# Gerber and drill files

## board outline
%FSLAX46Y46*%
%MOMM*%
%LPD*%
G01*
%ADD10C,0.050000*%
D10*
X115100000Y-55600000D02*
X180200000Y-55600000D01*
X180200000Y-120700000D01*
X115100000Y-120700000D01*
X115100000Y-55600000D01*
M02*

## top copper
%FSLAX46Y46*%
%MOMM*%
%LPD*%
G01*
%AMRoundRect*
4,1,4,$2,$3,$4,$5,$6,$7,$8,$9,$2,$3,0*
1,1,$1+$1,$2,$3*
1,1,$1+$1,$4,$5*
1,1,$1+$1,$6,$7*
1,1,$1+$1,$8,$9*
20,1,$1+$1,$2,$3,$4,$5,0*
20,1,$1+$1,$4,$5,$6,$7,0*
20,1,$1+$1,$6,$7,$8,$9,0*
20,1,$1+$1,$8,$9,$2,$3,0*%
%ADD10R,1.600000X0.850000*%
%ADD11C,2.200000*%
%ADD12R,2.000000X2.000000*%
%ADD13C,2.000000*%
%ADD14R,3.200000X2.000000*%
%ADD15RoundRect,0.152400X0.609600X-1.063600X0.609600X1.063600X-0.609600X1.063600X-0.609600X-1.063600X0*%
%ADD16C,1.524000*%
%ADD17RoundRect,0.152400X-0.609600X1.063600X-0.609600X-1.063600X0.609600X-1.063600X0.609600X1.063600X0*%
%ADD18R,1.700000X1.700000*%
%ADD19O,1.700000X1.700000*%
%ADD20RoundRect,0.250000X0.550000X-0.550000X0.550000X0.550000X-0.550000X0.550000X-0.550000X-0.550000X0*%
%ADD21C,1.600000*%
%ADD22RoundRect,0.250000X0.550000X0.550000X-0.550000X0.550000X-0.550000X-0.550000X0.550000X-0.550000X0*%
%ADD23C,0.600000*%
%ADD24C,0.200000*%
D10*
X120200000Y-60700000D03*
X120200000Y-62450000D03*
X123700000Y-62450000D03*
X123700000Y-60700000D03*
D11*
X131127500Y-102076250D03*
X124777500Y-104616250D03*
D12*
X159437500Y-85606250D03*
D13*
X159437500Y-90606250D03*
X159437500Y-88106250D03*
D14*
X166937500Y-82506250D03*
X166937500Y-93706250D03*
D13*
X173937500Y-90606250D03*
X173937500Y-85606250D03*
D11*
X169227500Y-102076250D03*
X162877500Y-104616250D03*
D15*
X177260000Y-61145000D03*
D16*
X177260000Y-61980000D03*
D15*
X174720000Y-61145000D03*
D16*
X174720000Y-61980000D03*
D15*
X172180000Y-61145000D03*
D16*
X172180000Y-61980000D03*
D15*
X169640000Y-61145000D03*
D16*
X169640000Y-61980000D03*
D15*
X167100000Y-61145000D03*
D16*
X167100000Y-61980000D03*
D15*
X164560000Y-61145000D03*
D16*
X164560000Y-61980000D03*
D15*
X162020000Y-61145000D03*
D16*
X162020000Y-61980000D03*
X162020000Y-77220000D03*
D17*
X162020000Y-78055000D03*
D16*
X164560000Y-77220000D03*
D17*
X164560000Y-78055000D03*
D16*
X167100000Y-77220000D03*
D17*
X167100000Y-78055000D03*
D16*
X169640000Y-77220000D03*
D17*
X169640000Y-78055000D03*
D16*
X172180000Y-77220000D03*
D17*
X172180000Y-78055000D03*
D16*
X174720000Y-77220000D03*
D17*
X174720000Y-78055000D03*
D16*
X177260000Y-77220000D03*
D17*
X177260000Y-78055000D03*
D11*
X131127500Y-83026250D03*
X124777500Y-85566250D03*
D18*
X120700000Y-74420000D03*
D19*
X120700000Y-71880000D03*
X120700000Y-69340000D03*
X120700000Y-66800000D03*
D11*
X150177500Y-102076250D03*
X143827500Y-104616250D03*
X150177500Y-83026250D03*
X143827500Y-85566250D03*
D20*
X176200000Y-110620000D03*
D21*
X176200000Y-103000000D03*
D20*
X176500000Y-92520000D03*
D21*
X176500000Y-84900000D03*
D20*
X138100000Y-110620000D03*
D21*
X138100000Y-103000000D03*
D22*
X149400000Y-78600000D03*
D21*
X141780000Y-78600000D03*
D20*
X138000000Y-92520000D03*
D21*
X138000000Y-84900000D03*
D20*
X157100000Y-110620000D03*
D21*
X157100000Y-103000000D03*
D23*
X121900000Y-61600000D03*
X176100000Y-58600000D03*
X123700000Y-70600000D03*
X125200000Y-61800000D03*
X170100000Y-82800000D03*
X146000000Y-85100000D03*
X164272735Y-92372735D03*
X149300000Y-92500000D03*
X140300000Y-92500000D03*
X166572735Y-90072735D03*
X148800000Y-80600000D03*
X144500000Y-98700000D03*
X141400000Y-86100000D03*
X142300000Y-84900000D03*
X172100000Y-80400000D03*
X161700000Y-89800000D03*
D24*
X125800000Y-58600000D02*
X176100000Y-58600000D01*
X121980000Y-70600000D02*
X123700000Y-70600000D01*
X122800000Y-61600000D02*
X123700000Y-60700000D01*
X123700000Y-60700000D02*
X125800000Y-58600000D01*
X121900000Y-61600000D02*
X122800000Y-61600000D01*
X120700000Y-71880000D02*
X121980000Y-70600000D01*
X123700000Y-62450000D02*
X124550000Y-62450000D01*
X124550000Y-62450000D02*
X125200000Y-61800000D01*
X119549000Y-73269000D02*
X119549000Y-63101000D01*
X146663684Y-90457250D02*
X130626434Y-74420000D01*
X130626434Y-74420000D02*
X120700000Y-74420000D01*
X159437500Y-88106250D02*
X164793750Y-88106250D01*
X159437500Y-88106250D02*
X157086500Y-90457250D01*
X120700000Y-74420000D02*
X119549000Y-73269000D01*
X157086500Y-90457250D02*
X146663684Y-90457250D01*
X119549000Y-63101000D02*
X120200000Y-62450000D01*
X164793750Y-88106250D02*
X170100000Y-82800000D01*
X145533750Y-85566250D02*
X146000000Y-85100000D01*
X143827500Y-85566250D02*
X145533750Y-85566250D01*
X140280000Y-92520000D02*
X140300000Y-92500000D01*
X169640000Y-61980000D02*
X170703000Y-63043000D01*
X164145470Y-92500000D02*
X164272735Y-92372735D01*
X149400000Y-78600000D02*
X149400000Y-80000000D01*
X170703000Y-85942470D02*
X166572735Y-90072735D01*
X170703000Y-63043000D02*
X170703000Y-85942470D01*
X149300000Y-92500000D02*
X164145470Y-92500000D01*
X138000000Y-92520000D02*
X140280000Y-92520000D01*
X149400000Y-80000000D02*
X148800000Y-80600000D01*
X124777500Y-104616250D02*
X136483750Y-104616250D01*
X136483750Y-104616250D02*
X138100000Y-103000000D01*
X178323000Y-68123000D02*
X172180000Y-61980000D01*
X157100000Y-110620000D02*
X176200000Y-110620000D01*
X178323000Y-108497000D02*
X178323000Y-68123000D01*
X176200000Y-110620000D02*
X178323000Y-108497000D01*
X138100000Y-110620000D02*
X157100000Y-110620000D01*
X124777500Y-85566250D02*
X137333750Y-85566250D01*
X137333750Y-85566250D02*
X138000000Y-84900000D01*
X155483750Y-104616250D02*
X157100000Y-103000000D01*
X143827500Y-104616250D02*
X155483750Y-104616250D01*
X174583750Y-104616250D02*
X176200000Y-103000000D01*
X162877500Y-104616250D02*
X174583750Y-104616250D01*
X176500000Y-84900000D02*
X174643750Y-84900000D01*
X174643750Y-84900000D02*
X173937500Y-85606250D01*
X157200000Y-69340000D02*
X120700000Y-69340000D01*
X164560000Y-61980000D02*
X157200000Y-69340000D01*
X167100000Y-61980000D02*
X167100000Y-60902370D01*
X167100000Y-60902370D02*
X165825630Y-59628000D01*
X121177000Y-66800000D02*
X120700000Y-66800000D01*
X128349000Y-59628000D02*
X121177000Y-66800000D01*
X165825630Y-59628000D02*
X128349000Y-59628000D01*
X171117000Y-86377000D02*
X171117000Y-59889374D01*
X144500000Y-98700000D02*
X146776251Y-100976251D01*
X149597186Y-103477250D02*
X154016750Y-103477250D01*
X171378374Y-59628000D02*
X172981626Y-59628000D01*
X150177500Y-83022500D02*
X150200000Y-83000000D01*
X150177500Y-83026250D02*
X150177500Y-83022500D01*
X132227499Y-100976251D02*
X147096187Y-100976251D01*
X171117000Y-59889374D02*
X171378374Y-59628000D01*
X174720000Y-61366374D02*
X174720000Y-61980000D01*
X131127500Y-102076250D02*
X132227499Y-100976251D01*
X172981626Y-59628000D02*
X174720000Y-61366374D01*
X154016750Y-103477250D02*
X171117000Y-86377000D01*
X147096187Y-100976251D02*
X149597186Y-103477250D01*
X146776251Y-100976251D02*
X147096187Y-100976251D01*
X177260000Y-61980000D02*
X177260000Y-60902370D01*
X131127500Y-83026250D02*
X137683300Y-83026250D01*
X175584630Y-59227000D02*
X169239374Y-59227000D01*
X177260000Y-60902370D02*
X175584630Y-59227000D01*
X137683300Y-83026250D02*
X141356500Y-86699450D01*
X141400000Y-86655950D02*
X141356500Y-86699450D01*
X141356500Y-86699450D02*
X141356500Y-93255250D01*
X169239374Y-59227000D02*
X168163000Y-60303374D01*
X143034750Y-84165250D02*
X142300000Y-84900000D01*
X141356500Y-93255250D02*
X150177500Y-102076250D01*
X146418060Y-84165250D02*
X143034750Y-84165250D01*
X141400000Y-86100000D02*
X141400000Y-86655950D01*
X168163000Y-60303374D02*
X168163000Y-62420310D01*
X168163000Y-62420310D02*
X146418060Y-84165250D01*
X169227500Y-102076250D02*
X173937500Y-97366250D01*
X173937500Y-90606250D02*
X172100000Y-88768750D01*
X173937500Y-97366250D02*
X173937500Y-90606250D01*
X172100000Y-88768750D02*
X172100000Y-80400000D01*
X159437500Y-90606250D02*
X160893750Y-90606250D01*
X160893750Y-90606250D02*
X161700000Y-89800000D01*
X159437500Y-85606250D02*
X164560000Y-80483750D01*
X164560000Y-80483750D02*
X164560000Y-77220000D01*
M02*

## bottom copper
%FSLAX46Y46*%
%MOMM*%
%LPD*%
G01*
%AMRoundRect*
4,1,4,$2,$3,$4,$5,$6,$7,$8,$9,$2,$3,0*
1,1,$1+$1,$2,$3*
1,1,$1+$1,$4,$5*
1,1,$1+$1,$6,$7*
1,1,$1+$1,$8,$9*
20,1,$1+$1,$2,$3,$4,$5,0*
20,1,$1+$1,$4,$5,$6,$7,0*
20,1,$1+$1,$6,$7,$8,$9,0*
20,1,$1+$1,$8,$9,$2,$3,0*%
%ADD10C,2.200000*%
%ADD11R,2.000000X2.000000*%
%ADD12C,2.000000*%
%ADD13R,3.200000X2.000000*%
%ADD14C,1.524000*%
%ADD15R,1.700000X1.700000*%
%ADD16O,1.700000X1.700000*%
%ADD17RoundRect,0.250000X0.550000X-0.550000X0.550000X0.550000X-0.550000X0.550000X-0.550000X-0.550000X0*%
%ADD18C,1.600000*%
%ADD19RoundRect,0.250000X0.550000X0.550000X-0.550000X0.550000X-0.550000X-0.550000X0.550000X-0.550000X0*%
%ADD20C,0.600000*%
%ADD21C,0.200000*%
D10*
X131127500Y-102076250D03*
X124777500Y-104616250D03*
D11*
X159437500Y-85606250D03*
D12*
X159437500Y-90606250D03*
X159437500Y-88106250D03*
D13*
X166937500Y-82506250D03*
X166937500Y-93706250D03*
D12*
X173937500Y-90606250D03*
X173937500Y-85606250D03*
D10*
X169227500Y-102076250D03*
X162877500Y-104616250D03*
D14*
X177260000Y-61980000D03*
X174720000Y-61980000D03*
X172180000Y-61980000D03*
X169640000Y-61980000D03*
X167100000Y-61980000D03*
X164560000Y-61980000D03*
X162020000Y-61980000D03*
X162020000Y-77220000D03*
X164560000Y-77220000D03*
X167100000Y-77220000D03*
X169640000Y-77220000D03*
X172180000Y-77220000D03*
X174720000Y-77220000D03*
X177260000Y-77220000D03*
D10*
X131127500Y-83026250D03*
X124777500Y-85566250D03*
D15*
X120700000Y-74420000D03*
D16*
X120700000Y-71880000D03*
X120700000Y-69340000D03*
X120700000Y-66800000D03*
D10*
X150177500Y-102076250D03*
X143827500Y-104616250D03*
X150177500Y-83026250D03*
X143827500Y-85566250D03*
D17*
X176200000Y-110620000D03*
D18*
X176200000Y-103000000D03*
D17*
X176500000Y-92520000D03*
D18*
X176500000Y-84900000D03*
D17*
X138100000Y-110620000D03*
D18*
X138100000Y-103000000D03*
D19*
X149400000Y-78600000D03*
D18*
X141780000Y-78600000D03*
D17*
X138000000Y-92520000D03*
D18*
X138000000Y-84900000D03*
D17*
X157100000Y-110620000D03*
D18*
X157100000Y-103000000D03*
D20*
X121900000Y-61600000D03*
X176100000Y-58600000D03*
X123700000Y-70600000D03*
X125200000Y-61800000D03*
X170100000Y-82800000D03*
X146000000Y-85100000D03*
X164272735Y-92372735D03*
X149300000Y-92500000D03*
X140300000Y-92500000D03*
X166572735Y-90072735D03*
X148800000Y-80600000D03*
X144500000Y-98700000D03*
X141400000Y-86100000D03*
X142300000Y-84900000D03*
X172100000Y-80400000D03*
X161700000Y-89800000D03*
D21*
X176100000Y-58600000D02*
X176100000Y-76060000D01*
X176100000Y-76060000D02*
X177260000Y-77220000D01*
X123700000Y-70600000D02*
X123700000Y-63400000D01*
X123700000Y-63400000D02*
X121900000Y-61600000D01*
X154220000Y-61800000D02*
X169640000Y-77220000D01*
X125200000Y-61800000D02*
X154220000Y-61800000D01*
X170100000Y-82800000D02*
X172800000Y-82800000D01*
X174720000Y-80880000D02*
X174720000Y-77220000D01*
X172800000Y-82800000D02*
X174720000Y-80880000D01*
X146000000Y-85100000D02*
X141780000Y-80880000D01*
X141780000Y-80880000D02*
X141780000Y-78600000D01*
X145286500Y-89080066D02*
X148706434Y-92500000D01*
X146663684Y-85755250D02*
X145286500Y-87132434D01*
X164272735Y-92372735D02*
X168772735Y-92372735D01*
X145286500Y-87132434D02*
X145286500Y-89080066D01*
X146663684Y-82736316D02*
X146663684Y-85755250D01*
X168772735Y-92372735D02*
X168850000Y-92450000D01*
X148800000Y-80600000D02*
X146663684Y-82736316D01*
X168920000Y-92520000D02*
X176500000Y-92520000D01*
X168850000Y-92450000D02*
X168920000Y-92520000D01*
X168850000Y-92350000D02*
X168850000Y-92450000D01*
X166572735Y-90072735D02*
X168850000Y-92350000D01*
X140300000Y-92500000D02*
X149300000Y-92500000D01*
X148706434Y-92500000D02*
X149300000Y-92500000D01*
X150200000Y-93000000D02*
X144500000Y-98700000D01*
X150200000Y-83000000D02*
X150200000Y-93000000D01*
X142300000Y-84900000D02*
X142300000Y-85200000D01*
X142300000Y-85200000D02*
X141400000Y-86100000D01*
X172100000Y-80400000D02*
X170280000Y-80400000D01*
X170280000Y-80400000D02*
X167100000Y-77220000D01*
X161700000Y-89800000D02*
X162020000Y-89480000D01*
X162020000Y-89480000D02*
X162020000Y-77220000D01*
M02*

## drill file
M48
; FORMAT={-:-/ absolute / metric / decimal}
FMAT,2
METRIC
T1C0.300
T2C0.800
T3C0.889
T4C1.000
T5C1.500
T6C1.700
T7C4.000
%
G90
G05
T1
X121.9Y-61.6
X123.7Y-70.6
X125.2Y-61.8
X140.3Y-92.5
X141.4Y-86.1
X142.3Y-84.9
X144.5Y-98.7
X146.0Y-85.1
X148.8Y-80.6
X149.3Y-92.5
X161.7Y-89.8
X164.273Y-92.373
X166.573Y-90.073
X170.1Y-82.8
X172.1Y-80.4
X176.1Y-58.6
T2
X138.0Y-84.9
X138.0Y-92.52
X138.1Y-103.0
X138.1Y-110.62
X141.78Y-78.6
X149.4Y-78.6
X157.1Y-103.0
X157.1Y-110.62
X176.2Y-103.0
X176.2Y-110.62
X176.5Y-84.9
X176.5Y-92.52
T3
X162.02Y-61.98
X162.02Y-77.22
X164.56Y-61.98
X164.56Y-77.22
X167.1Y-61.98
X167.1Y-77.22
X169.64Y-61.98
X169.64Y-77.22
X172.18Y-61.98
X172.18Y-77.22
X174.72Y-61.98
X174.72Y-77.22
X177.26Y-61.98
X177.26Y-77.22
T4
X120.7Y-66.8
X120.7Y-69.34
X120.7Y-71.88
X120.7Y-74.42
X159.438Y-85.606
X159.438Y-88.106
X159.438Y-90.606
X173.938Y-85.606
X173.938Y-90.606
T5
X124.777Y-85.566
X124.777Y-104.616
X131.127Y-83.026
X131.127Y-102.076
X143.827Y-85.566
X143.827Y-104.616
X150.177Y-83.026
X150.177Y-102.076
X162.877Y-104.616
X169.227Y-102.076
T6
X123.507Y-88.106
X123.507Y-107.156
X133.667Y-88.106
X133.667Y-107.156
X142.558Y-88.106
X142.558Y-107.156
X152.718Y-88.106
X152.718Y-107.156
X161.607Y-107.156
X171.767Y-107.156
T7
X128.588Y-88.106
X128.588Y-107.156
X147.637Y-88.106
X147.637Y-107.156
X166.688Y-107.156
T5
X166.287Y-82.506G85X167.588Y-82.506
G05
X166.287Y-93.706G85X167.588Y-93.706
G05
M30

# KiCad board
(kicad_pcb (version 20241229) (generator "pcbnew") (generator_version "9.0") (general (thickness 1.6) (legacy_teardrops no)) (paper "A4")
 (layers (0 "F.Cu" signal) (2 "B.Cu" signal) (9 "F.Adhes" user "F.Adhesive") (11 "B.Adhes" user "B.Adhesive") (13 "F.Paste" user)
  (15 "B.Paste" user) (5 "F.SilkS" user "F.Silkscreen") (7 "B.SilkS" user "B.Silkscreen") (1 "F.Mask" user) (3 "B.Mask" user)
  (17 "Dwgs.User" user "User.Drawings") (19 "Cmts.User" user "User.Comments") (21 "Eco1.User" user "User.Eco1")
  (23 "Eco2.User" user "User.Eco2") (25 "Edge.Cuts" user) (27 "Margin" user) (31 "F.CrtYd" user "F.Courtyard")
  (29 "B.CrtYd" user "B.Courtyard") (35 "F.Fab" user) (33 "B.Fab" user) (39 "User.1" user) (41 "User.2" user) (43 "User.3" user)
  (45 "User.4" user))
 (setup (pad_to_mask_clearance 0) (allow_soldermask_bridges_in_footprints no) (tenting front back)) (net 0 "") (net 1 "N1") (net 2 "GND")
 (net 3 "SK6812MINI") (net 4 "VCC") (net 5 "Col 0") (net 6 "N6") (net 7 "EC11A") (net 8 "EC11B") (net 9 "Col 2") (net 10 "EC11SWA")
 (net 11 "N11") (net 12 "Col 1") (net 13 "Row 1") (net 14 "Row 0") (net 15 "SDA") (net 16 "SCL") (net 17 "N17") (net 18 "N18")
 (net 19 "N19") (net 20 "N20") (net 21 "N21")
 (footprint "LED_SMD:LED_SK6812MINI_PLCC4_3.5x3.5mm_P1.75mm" (layer "F.Cu") (at 121.95 61.575)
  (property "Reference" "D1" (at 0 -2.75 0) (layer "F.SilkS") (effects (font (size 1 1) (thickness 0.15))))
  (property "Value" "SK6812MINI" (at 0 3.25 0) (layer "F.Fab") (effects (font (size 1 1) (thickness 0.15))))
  (pad "1" smd rect (at -1.75 -0.875) (size 1.6 0.85) (layers "F.Cu" "F.Mask" "F.Paste") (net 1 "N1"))
  (pad "2" smd rect (at -1.75 0.875) (size 1.6 0.85) (layers "F.Cu" "F.Mask" "F.Paste") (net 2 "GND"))
  (pad "3" smd rect (at 1.75 0.875) (size 1.6 0.85) (layers "F.Cu" "F.Mask" "F.Paste") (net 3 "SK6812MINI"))
  (pad "4" smd rect (at 1.75 -0.875) (size 1.6 0.85) (layers "F.Cu" "F.Mask" "F.Paste") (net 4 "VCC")))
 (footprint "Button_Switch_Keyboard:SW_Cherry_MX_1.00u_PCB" (layer "F.Cu") (at 131.1275 102.07625)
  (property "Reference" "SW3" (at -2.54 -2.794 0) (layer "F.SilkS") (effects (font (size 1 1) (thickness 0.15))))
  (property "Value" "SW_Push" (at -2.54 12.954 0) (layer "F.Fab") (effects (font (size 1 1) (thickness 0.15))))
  (pad "" np_thru_hole circle (at -7.62 5.08) (size 1.7 1.7) (drill 1.7) (layers "*.Cu" "*.Mask"))
  (pad "" np_thru_hole circle (at -2.54 5.08) (size 4 4) (drill 4) (layers "*.Cu" "*.Mask"))
  (pad "" np_thru_hole circle (at 2.54 5.08) (size 1.7 1.7) (drill 1.7) (layers "*.Cu" "*.Mask"))
  (pad "1" thru_hole circle (at 0 0) (size 2.2 2.2) (drill 1.5) (layers "*.Cu" "*.Mask") (remove_unused_layers no) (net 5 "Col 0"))
  (pad "2" thru_hole circle (at -6.35 2.54) (size 2.2 2.2) (drill 1.5) (layers "*.Cu" "*.Mask") (remove_unused_layers no) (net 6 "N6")))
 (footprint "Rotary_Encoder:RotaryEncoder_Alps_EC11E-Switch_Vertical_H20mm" (layer "F.Cu") (at 159.4375 85.60625)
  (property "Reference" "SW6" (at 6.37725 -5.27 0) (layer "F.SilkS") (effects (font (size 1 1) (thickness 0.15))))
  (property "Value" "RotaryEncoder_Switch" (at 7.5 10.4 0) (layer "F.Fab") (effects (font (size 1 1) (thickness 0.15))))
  (pad "A" thru_hole rect (at 0 0) (size 2 2) (drill 1) (layers "*.Cu" "*.Mask") (remove_unused_layers no) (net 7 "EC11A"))
  (pad "B" thru_hole circle (at 0 5) (size 2 2) (drill 1) (layers "*.Cu" "*.Mask") (remove_unused_layers no) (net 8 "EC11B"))
  (pad "C" thru_hole circle (at 0 2.5) (size 2 2) (drill 1) (layers "*.Cu" "*.Mask") (remove_unused_layers no) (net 2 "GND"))
  (pad "MP" thru_hole rect (at 7.5 -3.1) (size 3.2 2) (drill oval 2.8 1.5) (layers "*.Cu" "*.Mask") (remove_unused_layers no))
  (pad "MP" thru_hole rect (at 7.5 8.1) (size 3.2 2) (drill oval 2.8 1.5) (layers "*.Cu" "*.Mask") (remove_unused_layers no))
  (pad "S1" thru_hole circle (at 14.5 5) (size 2 2) (drill 1) (layers "*.Cu" "*.Mask") (remove_unused_layers no) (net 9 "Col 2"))
  (pad "S2" thru_hole circle (at 14.5 0) (size 2 2) (drill 1) (layers "*.Cu" "*.Mask") (remove_unused_layers no) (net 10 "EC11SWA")))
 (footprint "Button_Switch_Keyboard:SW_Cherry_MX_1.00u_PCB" (layer "F.Cu") (at 169.2275 102.07625)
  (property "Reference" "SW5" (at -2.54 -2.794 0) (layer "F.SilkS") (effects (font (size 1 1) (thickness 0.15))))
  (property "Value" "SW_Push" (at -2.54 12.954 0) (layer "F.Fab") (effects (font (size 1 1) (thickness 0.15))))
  (pad "" np_thru_hole circle (at -7.62 5.08) (size 1.7 1.7) (drill 1.7) (layers "*.Cu" "*.Mask"))
  (pad "" np_thru_hole circle (at -2.54 5.08) (size 4 4) (drill 4) (layers "*.Cu" "*.Mask"))
  (pad "" np_thru_hole circle (at 2.54 5.08) (size 1.7 1.7) (drill 1.7) (layers "*.Cu" "*.Mask"))
  (pad "1" thru_hole circle (at 0 0) (size 2.2 2.2) (drill 1.5) (layers "*.Cu" "*.Mask") (remove_unused_layers no) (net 9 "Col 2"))
  (pad "2" thru_hole circle (at -6.35 2.54) (size 2.2 2.2) (drill 1.5) (layers "*.Cu" "*.Mask") (remove_unused_layers no) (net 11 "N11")))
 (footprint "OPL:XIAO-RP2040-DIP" (layer "F.Cu") (at 169.64 69.6 -90)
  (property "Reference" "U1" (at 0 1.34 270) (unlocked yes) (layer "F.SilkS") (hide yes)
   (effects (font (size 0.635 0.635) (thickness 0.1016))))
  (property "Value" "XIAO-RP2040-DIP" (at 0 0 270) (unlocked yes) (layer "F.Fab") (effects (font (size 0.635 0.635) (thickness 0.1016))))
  (pad "1" smd roundrect (at -8.455 -7.62 90) (size 2.432 1.524) (layers "F.Cu" "F.Mask") (roundrect_rratio 0.1) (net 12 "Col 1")
   (thermal_bridge_angle 45))
  (pad "1" thru_hole circle (at -7.62 -7.62 90) (size 1.524 1.524) (drill 0.889) (layers "*.Cu" "*.Mask") (remove_unused_layers no)
   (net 12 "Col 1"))
  (pad "2" smd roundrect (at -8.455 -5.08 90) (size 2.432 1.524) (layers "F.Cu" "F.Mask") (roundrect_rratio 0.1) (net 5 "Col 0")
   (thermal_bridge_angle 45))
  (pad "2" thru_hole circle (at -7.62 -5.08 90) (size 1.524 1.524) (drill 0.889) (layers "*.Cu" "*.Mask") (remove_unused_layers no)
   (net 5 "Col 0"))
  (pad "3" smd roundrect (at -8.455 -2.54 90) (size 2.432 1.524) (layers "F.Cu" "F.Mask") (roundrect_rratio 0.1) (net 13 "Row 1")
   (thermal_bridge_angle 45))
  (pad "3" thru_hole circle (at -7.62 -2.54 90) (size 1.524 1.524) (drill 0.889) (layers "*.Cu" "*.Mask") (remove_unused_layers no)
   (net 13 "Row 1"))
  (pad "4" smd roundrect (at -8.455 0 90) (size 2.432 1.524) (layers "F.Cu" "F.Mask") (roundrect_rratio 0.1) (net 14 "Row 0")
   (thermal_bridge_angle 45))
  (pad "4" thru_hole circle (at -7.62 0 90) (size 1.524 1.524) (drill 0.889) (layers "*.Cu" "*.Mask") (remove_unused_layers no)
   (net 14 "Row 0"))
  (pad "5" smd roundrect (at -8.455 2.54 90) (size 2.432 1.524) (layers "F.Cu" "F.Mask") (roundrect_rratio 0.1) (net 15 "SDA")
   (thermal_bridge_angle 45))
  (pad "5" thru_hole circle (at -7.62 2.54 90) (size 1.524 1.524) (drill 0.889) (layers "*.Cu" "*.Mask") (remove_unused_layers no)
   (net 15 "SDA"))
  (pad "6" smd roundrect (at -8.455 5.08 90) (size 2.432 1.524) (layers "F.Cu" "F.Mask") (roundrect_rratio 0.1) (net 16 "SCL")
   (thermal_bridge_angle 45))
  (pad "6" thru_hole circle (at -7.62 5.08 90) (size 1.524 1.524) (drill 0.889) (layers "*.Cu" "*.Mask") (remove_unused_layers no)
   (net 16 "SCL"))
  (pad "7" smd roundrect (at -8.455 7.62 90) (size 2.432 1.524) (layers "F.Cu" "F.Mask") (roundrect_rratio 0.1) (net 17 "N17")
   (thermal_bridge_angle 45))
  (pad "7" thru_hole circle (at -7.62 7.62 90) (size 1.524 1.524) (drill 0.889) (layers "*.Cu" "*.Mask") (remove_unused_layers no)
   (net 17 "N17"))
  (pad "8" thru_hole circle (at 7.62 7.62 270) (size 1.524 1.524) (drill 0.889) (layers "*.Cu" "*.Mask") (remove_unused_layers no)
   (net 8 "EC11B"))
  (pad "8" smd roundrect (at 8.455 7.62 270) (size 2.432 1.524) (layers "F.Cu" "F.Mask") (roundrect_rratio 0.1) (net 8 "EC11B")
   (thermal_bridge_angle 45))
  (pad "9" thru_hole circle (at 7.62 5.08 270) (size 1.524 1.524) (drill 0.889) (layers "*.Cu" "*.Mask") (remove_unused_layers no)
   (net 7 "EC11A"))
  (pad "9" smd roundrect (at 8.455 5.08 270) (size 2.432 1.524) (layers "F.Cu" "F.Mask") (roundrect_rratio 0.1) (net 7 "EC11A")
   (thermal_bridge_angle 45))
  (pad "10" thru_hole circle (at 7.62 2.54 270) (size 1.524 1.524) (drill 0.889) (layers "*.Cu" "*.Mask") (remove_unused_layers no)
   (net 9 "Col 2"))
  (pad "10" smd roundrect (at 8.455 2.54 270) (size 2.432 1.524) (layers "F.Cu" "F.Mask") (roundrect_rratio 0.1) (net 9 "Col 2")
   (thermal_bridge_angle 45))
  (pad "11" thru_hole circle (at 7.62 0 270) (size 1.524 1.524) (drill 0.889) (layers "*.Cu" "*.Mask") (remove_unused_layers no)
   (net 3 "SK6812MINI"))
  (pad "11" smd roundrect (at 8.455 0 270) (size 2.432 1.524) (layers "F.Cu" "F.Mask") (roundrect_rratio 0.1) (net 3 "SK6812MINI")
   (thermal_bridge_angle 45))
  (pad "12" thru_hole circle (at 7.62 -2.54 270) (size 1.524 1.524) (drill 0.889) (layers "*.Cu" "*.Mask") (remove_unused_layers no)
   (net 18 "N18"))
  (pad "12" smd roundrect (at 8.455 -2.54 270) (size 2.432 1.524) (layers "F.Cu" "F.Mask") (roundrect_rratio 0.1) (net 18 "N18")
   (thermal_bridge_angle 45))
  (pad "13" thru_hole circle (at 7.62 -5.08 270) (size 1.524 1.524) (drill 0.889) (layers "*.Cu" "*.Mask") (remove_unused_layers no)
   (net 2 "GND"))
  (pad "13" smd roundrect (at 8.455 -5.08 270) (size 2.432 1.524) (layers "F.Cu" "F.Mask") (roundrect_rratio 0.1) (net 2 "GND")
   (thermal_bridge_angle 45))
  (pad "14" thru_hole circle (at 7.62 -7.62 270) (size 1.524 1.524) (drill 0.889) (layers "*.Cu" "*.Mask") (remove_unused_layers no)
   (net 4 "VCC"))
  (pad "14" smd roundrect (at 8.455 -7.62 270) (size 2.432 1.524) (layers "F.Cu" "F.Mask") (roundrect_rratio 0.1) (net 4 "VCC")
   (thermal_bridge_angle 45)))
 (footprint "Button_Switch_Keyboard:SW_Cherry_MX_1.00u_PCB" (layer "F.Cu") (at 131.1275 83.02625)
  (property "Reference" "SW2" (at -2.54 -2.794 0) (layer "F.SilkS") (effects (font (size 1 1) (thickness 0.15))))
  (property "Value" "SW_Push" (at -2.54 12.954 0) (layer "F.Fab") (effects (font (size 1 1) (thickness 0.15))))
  (pad "" np_thru_hole circle (at -7.62 5.08) (size 1.7 1.7) (drill 1.7) (layers "*.Cu" "*.Mask"))
  (pad "" np_thru_hole circle (at -2.54 5.08) (size 4 4) (drill 4) (layers "*.Cu" "*.Mask"))
  (pad "" np_thru_hole circle (at 2.54 5.08) (size 1.7 1.7) (drill 1.7) (layers "*.Cu" "*.Mask"))
  (pad "1" thru_hole circle (at 0 0) (size 2.2 2.2) (drill 1.5) (layers "*.Cu" "*.Mask") (remove_unused_layers no) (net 12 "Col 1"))
  (pad "2" thru_hole circle (at -6.35 2.54) (size 2.2 2.2) (drill 1.5) (layers "*.Cu" "*.Mask") (remove_unused_layers no) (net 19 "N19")))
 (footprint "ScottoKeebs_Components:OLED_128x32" (layer "F.Cu") (at 119.1 64.62)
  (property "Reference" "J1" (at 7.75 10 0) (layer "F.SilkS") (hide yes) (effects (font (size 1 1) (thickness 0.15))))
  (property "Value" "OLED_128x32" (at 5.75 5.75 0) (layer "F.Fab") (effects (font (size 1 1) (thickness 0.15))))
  (pad "1" thru_hole rect (at 1.6 9.8 180) (size 1.7 1.7) (drill 1) (layers "*.Cu" "*.Mask") (remove_unused_layers no) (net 2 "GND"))
  (pad "2" thru_hole oval (at 1.6 7.26 180) (size 1.7 1.7) (drill 1) (layers "*.Cu" "*.Mask") (remove_unused_layers no) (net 4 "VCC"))
  (pad "3" thru_hole oval (at 1.6 4.72 180) (size 1.7 1.7) (drill 1) (layers "*.Cu" "*.Mask") (remove_unused_layers no) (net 16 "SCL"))
  (pad "4" thru_hole oval (at 1.6 2.18 180) (size 1.7 1.7) (drill 1) (layers "*.Cu" "*.Mask") (remove_unused_layers no) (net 15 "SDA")))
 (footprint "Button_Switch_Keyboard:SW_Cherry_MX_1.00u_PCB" (layer "F.Cu") (at 150.1775 102.07625)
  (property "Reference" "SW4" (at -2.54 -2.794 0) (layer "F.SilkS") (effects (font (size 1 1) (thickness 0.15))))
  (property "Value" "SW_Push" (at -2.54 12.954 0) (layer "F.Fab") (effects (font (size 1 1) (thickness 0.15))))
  (pad "" np_thru_hole circle (at -7.62 5.08) (size 1.7 1.7) (drill 1.7) (layers "*.Cu" "*.Mask"))
  (pad "" np_thru_hole circle (at -2.54 5.08) (size 4 4) (drill 4) (layers "*.Cu" "*.Mask"))
  (pad "" np_thru_hole circle (at 2.54 5.08) (size 1.7 1.7) (drill 1.7) (layers "*.Cu" "*.Mask"))
  (pad "1" thru_hole circle (at 0 0) (size 2.2 2.2) (drill 1.5) (layers "*.Cu" "*.Mask") (remove_unused_layers no) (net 12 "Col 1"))
  (pad "2" thru_hole circle (at -6.35 2.54) (size 2.2 2.2) (drill 1.5) (layers "*.Cu" "*.Mask") (remove_unused_layers no) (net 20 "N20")))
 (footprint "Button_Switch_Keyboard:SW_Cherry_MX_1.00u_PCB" (layer "F.Cu") (at 150.1775 83.02625)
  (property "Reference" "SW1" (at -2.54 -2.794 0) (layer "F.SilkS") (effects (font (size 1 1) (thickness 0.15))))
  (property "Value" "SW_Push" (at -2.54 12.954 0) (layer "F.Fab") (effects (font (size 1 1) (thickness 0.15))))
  (pad "" np_thru_hole circle (at -7.62 5.08) (size 1.7 1.7) (drill 1.7) (layers "*.Cu" "*.Mask"))
  (pad "" np_thru_hole circle (at -2.54 5.08) (size 4 4) (drill 4) (layers "*.Cu" "*.Mask"))
  (pad "" np_thru_hole circle (at 2.54 5.08) (size 1.7 1.7) (drill 1.7) (layers "*.Cu" "*.Mask"))
  (pad "1" thru_hole circle (at 0 0) (size 2.2 2.2) (drill 1.5) (layers "*.Cu" "*.Mask") (remove_unused_layers no) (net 5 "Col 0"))
  (pad "2" thru_hole circle (at -6.35 2.54) (size 2.2 2.2) (drill 1.5) (layers "*.Cu" "*.Mask") (remove_unused_layers no) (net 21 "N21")))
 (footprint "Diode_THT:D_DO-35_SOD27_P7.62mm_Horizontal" (layer "B.Cu") (at 176.2 110.62 90)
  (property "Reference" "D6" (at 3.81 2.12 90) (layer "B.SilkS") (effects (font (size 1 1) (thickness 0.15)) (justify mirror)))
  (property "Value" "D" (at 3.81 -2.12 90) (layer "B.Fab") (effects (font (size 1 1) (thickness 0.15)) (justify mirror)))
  (pad "1" thru_hole roundrect (at 0 0 90) (size 1.6 1.6) (drill 0.8) (layers "*.Cu" "*.Mask") (remove_unused_layers no)
   (roundrect_rratio 0.15625) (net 13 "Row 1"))
  (pad "2" thru_hole circle (at 7.62 0 90) (size 1.6 1.6) (drill 0.8) (layers "*.Cu" "*.Mask") (remove_unused_layers no) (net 11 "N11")))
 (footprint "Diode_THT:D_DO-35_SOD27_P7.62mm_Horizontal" (layer "B.Cu") (at 176.5 92.52 90)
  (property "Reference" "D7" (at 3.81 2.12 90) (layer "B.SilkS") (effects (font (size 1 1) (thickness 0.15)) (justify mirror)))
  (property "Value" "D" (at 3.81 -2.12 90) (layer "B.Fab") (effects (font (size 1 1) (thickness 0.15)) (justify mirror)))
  (pad "1" thru_hole roundrect (at 0 0 90) (size 1.6 1.6) (drill 0.8) (layers "*.Cu" "*.Mask") (remove_unused_layers no)
   (roundrect_rratio 0.15625) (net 14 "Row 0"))
  (pad "2" thru_hole circle (at 7.62 0 90) (size 1.6 1.6) (drill 0.8) (layers "*.Cu" "*.Mask") (remove_unused_layers no) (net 10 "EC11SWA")))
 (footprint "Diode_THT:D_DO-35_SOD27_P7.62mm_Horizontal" (layer "B.Cu") (at 138.1 110.62 90)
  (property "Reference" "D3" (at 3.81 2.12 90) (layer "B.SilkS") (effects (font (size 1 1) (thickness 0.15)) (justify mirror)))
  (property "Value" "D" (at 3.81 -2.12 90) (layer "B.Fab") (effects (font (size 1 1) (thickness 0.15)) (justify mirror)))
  (pad "1" thru_hole roundrect (at 0 0 90) (size 1.6 1.6) (drill 0.8) (layers "*.Cu" "*.Mask") (remove_unused_layers no)
   (roundrect_rratio 0.15625) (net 13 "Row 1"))
  (pad "2" thru_hole circle (at 7.62 0 90) (size 1.6 1.6) (drill 0.8) (layers "*.Cu" "*.Mask") (remove_unused_layers no) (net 6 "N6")))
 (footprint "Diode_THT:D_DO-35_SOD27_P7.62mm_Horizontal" (layer "B.Cu") (at 149.4 78.6 180)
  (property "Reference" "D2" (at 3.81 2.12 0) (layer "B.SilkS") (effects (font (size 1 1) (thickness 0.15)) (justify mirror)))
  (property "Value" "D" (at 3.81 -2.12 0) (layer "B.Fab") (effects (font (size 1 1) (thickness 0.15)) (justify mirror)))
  (pad "1" thru_hole roundrect (at 0 0 180) (size 1.6 1.6) (drill 0.8) (layers "*.Cu" "*.Mask") (remove_unused_layers no)
   (roundrect_rratio 0.15625) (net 14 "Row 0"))
  (pad "2" thru_hole circle (at 7.62 0 180) (size 1.6 1.6) (drill 0.8) (layers "*.Cu" "*.Mask") (remove_unused_layers no) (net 21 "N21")))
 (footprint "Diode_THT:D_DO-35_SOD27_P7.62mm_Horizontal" (layer "B.Cu") (at 138 92.52 90)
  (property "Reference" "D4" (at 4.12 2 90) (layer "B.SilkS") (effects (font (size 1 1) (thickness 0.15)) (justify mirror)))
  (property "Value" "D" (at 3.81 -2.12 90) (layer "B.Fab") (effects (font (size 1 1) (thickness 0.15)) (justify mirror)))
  (pad "1" thru_hole roundrect (at 0 0 90) (size 1.6 1.6) (drill 0.8) (layers "*.Cu" "*.Mask") (remove_unused_layers no)
   (roundrect_rratio 0.15625) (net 14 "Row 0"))
  (pad "2" thru_hole circle (at 7.62 0 90) (size 1.6 1.6) (drill 0.8) (layers "*.Cu" "*.Mask") (remove_unused_layers no) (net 19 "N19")))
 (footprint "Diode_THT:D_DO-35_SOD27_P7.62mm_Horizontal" (layer "B.Cu") (at 157.1 110.62 90)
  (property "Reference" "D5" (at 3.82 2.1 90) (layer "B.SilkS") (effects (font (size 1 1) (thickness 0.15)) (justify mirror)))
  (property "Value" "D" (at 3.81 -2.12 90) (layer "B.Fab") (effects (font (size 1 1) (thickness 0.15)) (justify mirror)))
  (pad "1" thru_hole roundrect (at 0 0 90) (size 1.6 1.6) (drill 0.8) (layers "*.Cu" "*.Mask") (remove_unused_layers no)
   (roundrect_rratio 0.15625) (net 13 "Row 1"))
  (pad "2" thru_hole circle (at 7.62 0 90) (size 1.6 1.6) (drill 0.8) (layers "*.Cu" "*.Mask") (remove_unused_layers no) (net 20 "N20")))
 (gr_rect (start 115.1 55.6) (end 180.2 120.7) (stroke (width 0.05) (type default)) (fill no) (layer "Edge.Cuts"))
 (segment (start 125.8 58.6) (end 176.1 58.6) (width 0.2) (layer "F.Cu") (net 4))
 (segment (start 121.98 70.6) (end 123.7 70.6) (width 0.2) (layer "F.Cu") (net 4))
 (segment (start 122.8 61.6) (end 123.7 60.7) (width 0.2) (layer "F.Cu") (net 4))
 (segment (start 123.7 60.7) (end 125.8 58.6) (width 0.2) (layer "F.Cu") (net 4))
 (segment (start 121.9 61.6) (end 122.8 61.6) (width 0.2) (layer "F.Cu") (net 4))
 (segment (start 120.7 71.88) (end 121.98 70.6) (width 0.2) (layer "F.Cu") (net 4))
 (via (at 121.9 61.6) (size 0.6) (drill 0.3) (layers "F.Cu" "B.Cu") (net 4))
 (via (at 176.1 58.6) (size 0.6) (drill 0.3) (layers "F.Cu" "B.Cu") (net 4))
 (via (at 123.7 70.6) (size 0.6) (drill 0.3) (layers "F.Cu" "B.Cu") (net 4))
 (segment (start 176.1 58.6) (end 176.1 76.06) (width 0.2) (layer "B.Cu") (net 4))
 (segment (start 176.1 76.06) (end 177.26 77.22) (width 0.2) (layer "B.Cu") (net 4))
 (segment (start 123.7 70.6) (end 123.7 63.4) (width 0.2) (layer "B.Cu") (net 4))
 (segment (start 123.7 63.4) (end 121.9 61.6) (width 0.2) (layer "B.Cu") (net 4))
 (segment (start 123.7 62.45) (end 124.55 62.45) (width 0.2) (layer "F.Cu") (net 3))
 (segment (start 124.55 62.45) (end 125.2 61.8) (width 0.2) (layer "F.Cu") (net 3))
 (via (at 125.2 61.8) (size 0.6) (drill 0.3) (layers "F.Cu" "B.Cu") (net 3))
 (segment (start 154.22 61.8) (end 169.64 77.22) (width 0.2) (layer "B.Cu") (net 3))
 (segment (start 125.2 61.8) (end 154.22 61.8) (width 0.2) (layer "B.Cu") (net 3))
 (segment (start 119.549 73.269) (end 119.549 63.101) (width 0.2) (layer "F.Cu") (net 2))
 (segment (start 146.663684 90.45725) (end 130.626434 74.42) (width 0.2) (layer "F.Cu") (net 2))
 (segment (start 130.626434 74.42) (end 120.7 74.42) (width 0.2) (layer "F.Cu") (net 2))
 (segment (start 159.4375 88.10625) (end 164.79375 88.10625) (width 0.2) (layer "F.Cu") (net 2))
 (segment (start 159.4375 88.10625) (end 157.0865 90.45725) (width 0.2) (layer "F.Cu") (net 2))
 (segment (start 120.7 74.42) (end 119.549 73.269) (width 0.2) (layer "F.Cu") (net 2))
 (segment (start 157.0865 90.45725) (end 146.663684 90.45725) (width 0.2) (layer "F.Cu") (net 2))
 (segment (start 119.549 63.101) (end 120.2 62.45) (width 0.2) (layer "F.Cu") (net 2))
 (segment (start 164.79375 88.10625) (end 170.1 82.8) (width 0.2) (layer "F.Cu") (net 2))
 (via (at 170.1 82.8) (size 0.6) (drill 0.3) (layers "F.Cu" "B.Cu") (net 2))
 (segment (start 170.1 82.8) (end 172.8 82.8) (width 0.2) (layer "B.Cu") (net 2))
 (segment (start 174.72 80.88) (end 174.72 77.22) (width 0.2) (layer "B.Cu") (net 2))
 (segment (start 172.8 82.8) (end 174.72 80.88) (width 0.2) (layer "B.Cu") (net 2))
 (segment (start 145.53375 85.56625) (end 146 85.1) (width 0.2) (layer "F.Cu") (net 21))
 (segment (start 143.8275 85.56625) (end 145.53375 85.56625) (width 0.2) (layer "F.Cu") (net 21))
 (via (at 146 85.1) (size 0.6) (drill 0.3) (layers "F.Cu" "B.Cu") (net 21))
 (segment (start 146 85.1) (end 141.78 80.88) (width 0.2) (layer "B.Cu") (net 21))
 (segment (start 141.78 80.88) (end 141.78 78.6) (width 0.2) (layer "B.Cu") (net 21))
 (segment (start 140.28 92.52) (end 140.3 92.5) (width 0.2) (layer "F.Cu") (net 14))
 (segment (start 169.64 61.98) (end 170.703 63.043) (width 0.2) (layer "F.Cu") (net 14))
 (segment (start 164.14547 92.5) (end 164.272735 92.372735) (width 0.2) (layer "F.Cu") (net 14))
 (segment (start 149.4 78.6) (end 149.4 80) (width 0.2) (layer "F.Cu") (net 14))
 (segment (start 170.703 85.94247) (end 166.572735 90.072735) (width 0.2) (layer "F.Cu") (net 14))
 (segment (start 170.703 63.043) (end 170.703 85.94247) (width 0.2) (layer "F.Cu") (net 14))
 (segment (start 149.3 92.5) (end 164.14547 92.5) (width 0.2) (layer "F.Cu") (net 14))
 (segment (start 138 92.52) (end 140.28 92.52) (width 0.2) (layer "F.Cu") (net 14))
 (segment (start 149.4 80) (end 148.8 80.6) (width 0.2) (layer "F.Cu") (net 14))
 (via (at 164.272735 92.372735) (size 0.6) (drill 0.3) (layers "F.Cu" "B.Cu") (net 14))
 (via (at 149.3 92.5) (size 0.6) (drill 0.3) (layers "F.Cu" "B.Cu") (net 14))
 (via (at 140.3 92.5) (size 0.6) (drill 0.3) (layers "F.Cu" "B.Cu") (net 14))
 (via (at 166.572735 90.072735) (size 0.6) (drill 0.3) (layers "F.Cu" "B.Cu") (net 14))
 (via (at 148.8 80.6) (size 0.6) (drill 0.3) (layers "F.Cu" "B.Cu") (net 14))
 (segment (start 145.2865 89.080066) (end 148.706434 92.5) (width 0.2) (layer "B.Cu") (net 14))
 (segment (start 146.663684 85.75525) (end 145.2865 87.132434) (width 0.2) (layer "B.Cu") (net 14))
 (segment (start 164.272735 92.372735) (end 168.772735 92.372735) (width 0.2) (layer "B.Cu") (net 14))
 (segment (start 145.2865 87.132434) (end 145.2865 89.080066) (width 0.2) (layer "B.Cu") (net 14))
 (segment (start 146.663684 82.736316) (end 146.663684 85.75525) (width 0.2) (layer "B.Cu") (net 14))
 (segment (start 168.772735 92.372735) (end 168.85 92.45) (width 0.2) (layer "B.Cu") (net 14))
 (segment (start 148.8 80.6) (end 146.663684 82.736316) (width 0.2) (layer "B.Cu") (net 14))
 (segment (start 168.92 92.52) (end 176.5 92.52) (width 0.2) (layer "B.Cu") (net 14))
 (segment (start 168.85 92.45) (end 168.92 92.52) (width 0.2) (layer "B.Cu") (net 14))
 (segment (start 168.85 92.35) (end 168.85 92.45) (width 0.2) (layer "B.Cu") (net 14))
 (segment (start 166.572735 90.072735) (end 168.85 92.35) (width 0.2) (layer "B.Cu") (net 14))
 (segment (start 140.3 92.5) (end 149.3 92.5) (width 0.2) (layer "B.Cu") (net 14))
 (segment (start 148.706434 92.5) (end 149.3 92.5) (width 0.2) (layer "B.Cu") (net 14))
 (segment (start 124.7775 104.61625) (end 136.48375 104.61625) (width 0.2) (layer "F.Cu") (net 6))
 (segment (start 136.48375 104.61625) (end 138.1 103) (width 0.2) (layer "F.Cu") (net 6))
 (segment (start 178.323 68.123) (end 172.18 61.98) (width 0.2) (layer "F.Cu") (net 13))
 (segment (start 157.1 110.62) (end 176.2 110.62) (width 0.2) (layer "F.Cu") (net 13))
 (segment (start 178.323 108.497) (end 178.323 68.123) (width 0.2) (layer "F.Cu") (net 13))
 (segment (start 176.2 110.62) (end 178.323 108.497) (width 0.2) (layer "F.Cu") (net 13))
 (segment (start 138.1 110.62) (end 157.1 110.62) (width 0.2) (layer "F.Cu") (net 13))
 (segment (start 124.7775 85.56625) (end 137.33375 85.56625) (width 0.2) (layer "F.Cu") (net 19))
 (segment (start 137.33375 85.56625) (end 138 84.9) (width 0.2) (layer "F.Cu") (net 19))
 (segment (start 155.48375 104.61625) (end 157.1 103) (width 0.2) (layer "F.Cu") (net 20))
 (segment (start 143.8275 104.61625) (end 155.48375 104.61625) (width 0.2) (layer "F.Cu") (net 20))
 (segment (start 174.58375 104.61625) (end 176.2 103) (width 0.2) (layer "F.Cu") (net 11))
 (segment (start 162.8775 104.61625) (end 174.58375 104.61625) (width 0.2) (layer "F.Cu") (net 11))
 (segment (start 176.5 84.9) (end 174.64375 84.9) (width 0.2) (layer "F.Cu") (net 10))
 (segment (start 174.64375 84.9) (end 173.9375 85.60625) (width 0.2) (layer "F.Cu") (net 10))
 (segment (start 157.2 69.34) (end 120.7 69.34) (width 0.2) (layer "F.Cu") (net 16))
 (segment (start 164.56 61.98) (end 157.2 69.34) (width 0.2) (layer "F.Cu") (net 16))
 (segment (start 167.1 61.98) (end 167.1 60.90237) (width 0.2) (layer "F.Cu") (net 15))
 (segment (start 167.1 60.90237) (end 165.82563 59.628) (width 0.2) (layer "F.Cu") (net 15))
 (segment (start 121.177 66.8) (end 120.7 66.8) (width 0.2) (layer "F.Cu") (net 15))
 (segment (start 128.349 59.628) (end 121.177 66.8) (width 0.2) (layer "F.Cu") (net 15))
 (segment (start 165.82563 59.628) (end 128.349 59.628) (width 0.2) (layer "F.Cu") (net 15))
 (segment (start 171.117 86.377) (end 171.117 59.889374) (width 0.2) (layer "F.Cu") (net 5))
 (segment (start 144.5 98.7) (end 146.776251 100.976251) (width 0.2) (layer "F.Cu") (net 5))
 (segment (start 149.597186 103.47725) (end 154.01675 103.47725) (width 0.2) (layer "F.Cu") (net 5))
 (segment (start 171.378374 59.628) (end 172.981626 59.628) (width 0.2) (layer "F.Cu") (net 5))
 (segment (start 150.1775 83.0225) (end 150.2 83) (width 0.2) (layer "F.Cu") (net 5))
 (segment (start 150.1775 83.02625) (end 150.1775 83.0225) (width 0.2) (layer "F.Cu") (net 5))
 (segment (start 132.227499 100.976251) (end 147.096187 100.976251) (width 0.2) (layer "F.Cu") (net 5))
 (segment (start 171.117 59.889374) (end 171.378374 59.628) (width 0.2) (layer "F.Cu") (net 5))
 (segment (start 174.72 61.366374) (end 174.72 61.98) (width 0.2) (layer "F.Cu") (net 5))
 (segment (start 131.1275 102.07625) (end 132.227499 100.976251) (width 0.2) (layer "F.Cu") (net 5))
 (segment (start 172.981626 59.628) (end 174.72 61.366374) (width 0.2) (layer "F.Cu") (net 5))
 (segment (start 154.01675 103.47725) (end 171.117 86.377) (width 0.2) (layer "F.Cu") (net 5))
 (segment (start 147.096187 100.976251) (end 149.597186 103.47725) (width 0.2) (layer "F.Cu") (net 5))
 (segment (start 146.776251 100.976251) (end 147.096187 100.976251) (width 0.2) (layer "F.Cu") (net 5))
 (via (at 144.5 98.7) (size 0.6) (drill 0.3) (layers "F.Cu" "B.Cu") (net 5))
 (segment (start 150.2 93) (end 144.5 98.7) (width 0.2) (layer "B.Cu") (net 5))
 (segment (start 150.2 83) (end 150.2 93) (width 0.2) (layer "B.Cu") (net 5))
 (segment (start 177.26 61.98) (end 177.26 60.90237) (width 0.2) (layer "F.Cu") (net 12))
 (segment (start 131.1275 83.02625) (end 137.6833 83.02625) (width 0.2) (layer "F.Cu") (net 12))
 (segment (start 175.58463 59.227) (end 169.239374 59.227) (width 0.2) (layer "F.Cu") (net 12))
 (segment (start 177.26 60.90237) (end 175.58463 59.227) (width 0.2) (layer "F.Cu") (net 12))
 (segment (start 137.6833 83.02625) (end 141.3565 86.69945) (width 0.2) (layer "F.Cu") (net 12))
 (segment (start 141.4 86.65595) (end 141.3565 86.69945) (width 0.2) (layer "F.Cu") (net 12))
 (segment (start 141.3565 86.69945) (end 141.3565 93.25525) (width 0.2) (layer "F.Cu") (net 12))
 (segment (start 169.239374 59.227) (end 168.163 60.303374) (width 0.2) (layer "F.Cu") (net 12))
 (segment (start 143.03475 84.16525) (end 142.3 84.9) (width 0.2) (layer "F.Cu") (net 12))
 (segment (start 141.3565 93.25525) (end 150.1775 102.07625) (width 0.2) (layer "F.Cu") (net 12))
 (segment (start 146.41806 84.16525) (end 143.03475 84.16525) (width 0.2) (layer "F.Cu") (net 12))
 (segment (start 141.4 86.1) (end 141.4 86.65595) (width 0.2) (layer "F.Cu") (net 12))
 (segment (start 168.163 60.303374) (end 168.163 62.42031) (width 0.2) (layer "F.Cu") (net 12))
 (segment (start 168.163 62.42031) (end 146.41806 84.16525) (width 0.2) (layer "F.Cu") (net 12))
 (via (at 141.4 86.1) (size 0.6) (drill 0.3) (layers "F.Cu" "B.Cu") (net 12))
 (via (at 142.3 84.9) (size 0.6) (drill 0.3) (layers "F.Cu" "B.Cu") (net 12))
 (segment (start 142.3 84.9) (end 142.3 85.2) (width 0.2) (layer "B.Cu") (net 12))
 (segment (start 142.3 85.2) (end 141.4 86.1) (width 0.2) (layer "B.Cu") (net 12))
 (segment (start 169.2275 102.07625) (end 173.9375 97.36625) (width 0.2) (layer "F.Cu") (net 9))
 (segment (start 173.9375 90.60625) (end 172.1 88.76875) (width 0.2) (layer "F.Cu") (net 9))
 (segment (start 173.9375 97.36625) (end 173.9375 90.60625) (width 0.2) (layer "F.Cu") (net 9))
 (segment (start 172.1 88.76875) (end 172.1 80.4) (width 0.2) (layer "F.Cu") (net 9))
 (via (at 172.1 80.4) (size 0.6) (drill 0.3) (layers "F.Cu" "B.Cu") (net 9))
 (segment (start 172.1 80.4) (end 170.28 80.4) (width 0.2) (layer "B.Cu") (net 9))
 (segment (start 170.28 80.4) (end 167.1 77.22) (width 0.2) (layer "B.Cu") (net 9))
 (segment (start 159.4375 90.60625) (end 160.89375 90.60625) (width 0.2) (layer "F.Cu") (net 8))
 (segment (start 160.89375 90.60625) (end 161.7 89.8) (width 0.2) (layer "F.Cu") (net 8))
 (via (at 161.7 89.8) (size 0.6) (drill 0.3) (layers "F.Cu" "B.Cu") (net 8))
 (segment (start 161.7 89.8) (end 162.02 89.48) (width 0.2) (layer "B.Cu") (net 8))
 (segment (start 162.02 89.48) (end 162.02 77.22) (width 0.2) (layer "B.Cu") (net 8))
 (segment (start 159.4375 85.60625) (end 164.56 80.48375) (width 0.2) (layer "F.Cu") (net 7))
 (segment (start 164.56 80.48375) (end 164.56 77.22) (width 0.2) (layer "F.Cu") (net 7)))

